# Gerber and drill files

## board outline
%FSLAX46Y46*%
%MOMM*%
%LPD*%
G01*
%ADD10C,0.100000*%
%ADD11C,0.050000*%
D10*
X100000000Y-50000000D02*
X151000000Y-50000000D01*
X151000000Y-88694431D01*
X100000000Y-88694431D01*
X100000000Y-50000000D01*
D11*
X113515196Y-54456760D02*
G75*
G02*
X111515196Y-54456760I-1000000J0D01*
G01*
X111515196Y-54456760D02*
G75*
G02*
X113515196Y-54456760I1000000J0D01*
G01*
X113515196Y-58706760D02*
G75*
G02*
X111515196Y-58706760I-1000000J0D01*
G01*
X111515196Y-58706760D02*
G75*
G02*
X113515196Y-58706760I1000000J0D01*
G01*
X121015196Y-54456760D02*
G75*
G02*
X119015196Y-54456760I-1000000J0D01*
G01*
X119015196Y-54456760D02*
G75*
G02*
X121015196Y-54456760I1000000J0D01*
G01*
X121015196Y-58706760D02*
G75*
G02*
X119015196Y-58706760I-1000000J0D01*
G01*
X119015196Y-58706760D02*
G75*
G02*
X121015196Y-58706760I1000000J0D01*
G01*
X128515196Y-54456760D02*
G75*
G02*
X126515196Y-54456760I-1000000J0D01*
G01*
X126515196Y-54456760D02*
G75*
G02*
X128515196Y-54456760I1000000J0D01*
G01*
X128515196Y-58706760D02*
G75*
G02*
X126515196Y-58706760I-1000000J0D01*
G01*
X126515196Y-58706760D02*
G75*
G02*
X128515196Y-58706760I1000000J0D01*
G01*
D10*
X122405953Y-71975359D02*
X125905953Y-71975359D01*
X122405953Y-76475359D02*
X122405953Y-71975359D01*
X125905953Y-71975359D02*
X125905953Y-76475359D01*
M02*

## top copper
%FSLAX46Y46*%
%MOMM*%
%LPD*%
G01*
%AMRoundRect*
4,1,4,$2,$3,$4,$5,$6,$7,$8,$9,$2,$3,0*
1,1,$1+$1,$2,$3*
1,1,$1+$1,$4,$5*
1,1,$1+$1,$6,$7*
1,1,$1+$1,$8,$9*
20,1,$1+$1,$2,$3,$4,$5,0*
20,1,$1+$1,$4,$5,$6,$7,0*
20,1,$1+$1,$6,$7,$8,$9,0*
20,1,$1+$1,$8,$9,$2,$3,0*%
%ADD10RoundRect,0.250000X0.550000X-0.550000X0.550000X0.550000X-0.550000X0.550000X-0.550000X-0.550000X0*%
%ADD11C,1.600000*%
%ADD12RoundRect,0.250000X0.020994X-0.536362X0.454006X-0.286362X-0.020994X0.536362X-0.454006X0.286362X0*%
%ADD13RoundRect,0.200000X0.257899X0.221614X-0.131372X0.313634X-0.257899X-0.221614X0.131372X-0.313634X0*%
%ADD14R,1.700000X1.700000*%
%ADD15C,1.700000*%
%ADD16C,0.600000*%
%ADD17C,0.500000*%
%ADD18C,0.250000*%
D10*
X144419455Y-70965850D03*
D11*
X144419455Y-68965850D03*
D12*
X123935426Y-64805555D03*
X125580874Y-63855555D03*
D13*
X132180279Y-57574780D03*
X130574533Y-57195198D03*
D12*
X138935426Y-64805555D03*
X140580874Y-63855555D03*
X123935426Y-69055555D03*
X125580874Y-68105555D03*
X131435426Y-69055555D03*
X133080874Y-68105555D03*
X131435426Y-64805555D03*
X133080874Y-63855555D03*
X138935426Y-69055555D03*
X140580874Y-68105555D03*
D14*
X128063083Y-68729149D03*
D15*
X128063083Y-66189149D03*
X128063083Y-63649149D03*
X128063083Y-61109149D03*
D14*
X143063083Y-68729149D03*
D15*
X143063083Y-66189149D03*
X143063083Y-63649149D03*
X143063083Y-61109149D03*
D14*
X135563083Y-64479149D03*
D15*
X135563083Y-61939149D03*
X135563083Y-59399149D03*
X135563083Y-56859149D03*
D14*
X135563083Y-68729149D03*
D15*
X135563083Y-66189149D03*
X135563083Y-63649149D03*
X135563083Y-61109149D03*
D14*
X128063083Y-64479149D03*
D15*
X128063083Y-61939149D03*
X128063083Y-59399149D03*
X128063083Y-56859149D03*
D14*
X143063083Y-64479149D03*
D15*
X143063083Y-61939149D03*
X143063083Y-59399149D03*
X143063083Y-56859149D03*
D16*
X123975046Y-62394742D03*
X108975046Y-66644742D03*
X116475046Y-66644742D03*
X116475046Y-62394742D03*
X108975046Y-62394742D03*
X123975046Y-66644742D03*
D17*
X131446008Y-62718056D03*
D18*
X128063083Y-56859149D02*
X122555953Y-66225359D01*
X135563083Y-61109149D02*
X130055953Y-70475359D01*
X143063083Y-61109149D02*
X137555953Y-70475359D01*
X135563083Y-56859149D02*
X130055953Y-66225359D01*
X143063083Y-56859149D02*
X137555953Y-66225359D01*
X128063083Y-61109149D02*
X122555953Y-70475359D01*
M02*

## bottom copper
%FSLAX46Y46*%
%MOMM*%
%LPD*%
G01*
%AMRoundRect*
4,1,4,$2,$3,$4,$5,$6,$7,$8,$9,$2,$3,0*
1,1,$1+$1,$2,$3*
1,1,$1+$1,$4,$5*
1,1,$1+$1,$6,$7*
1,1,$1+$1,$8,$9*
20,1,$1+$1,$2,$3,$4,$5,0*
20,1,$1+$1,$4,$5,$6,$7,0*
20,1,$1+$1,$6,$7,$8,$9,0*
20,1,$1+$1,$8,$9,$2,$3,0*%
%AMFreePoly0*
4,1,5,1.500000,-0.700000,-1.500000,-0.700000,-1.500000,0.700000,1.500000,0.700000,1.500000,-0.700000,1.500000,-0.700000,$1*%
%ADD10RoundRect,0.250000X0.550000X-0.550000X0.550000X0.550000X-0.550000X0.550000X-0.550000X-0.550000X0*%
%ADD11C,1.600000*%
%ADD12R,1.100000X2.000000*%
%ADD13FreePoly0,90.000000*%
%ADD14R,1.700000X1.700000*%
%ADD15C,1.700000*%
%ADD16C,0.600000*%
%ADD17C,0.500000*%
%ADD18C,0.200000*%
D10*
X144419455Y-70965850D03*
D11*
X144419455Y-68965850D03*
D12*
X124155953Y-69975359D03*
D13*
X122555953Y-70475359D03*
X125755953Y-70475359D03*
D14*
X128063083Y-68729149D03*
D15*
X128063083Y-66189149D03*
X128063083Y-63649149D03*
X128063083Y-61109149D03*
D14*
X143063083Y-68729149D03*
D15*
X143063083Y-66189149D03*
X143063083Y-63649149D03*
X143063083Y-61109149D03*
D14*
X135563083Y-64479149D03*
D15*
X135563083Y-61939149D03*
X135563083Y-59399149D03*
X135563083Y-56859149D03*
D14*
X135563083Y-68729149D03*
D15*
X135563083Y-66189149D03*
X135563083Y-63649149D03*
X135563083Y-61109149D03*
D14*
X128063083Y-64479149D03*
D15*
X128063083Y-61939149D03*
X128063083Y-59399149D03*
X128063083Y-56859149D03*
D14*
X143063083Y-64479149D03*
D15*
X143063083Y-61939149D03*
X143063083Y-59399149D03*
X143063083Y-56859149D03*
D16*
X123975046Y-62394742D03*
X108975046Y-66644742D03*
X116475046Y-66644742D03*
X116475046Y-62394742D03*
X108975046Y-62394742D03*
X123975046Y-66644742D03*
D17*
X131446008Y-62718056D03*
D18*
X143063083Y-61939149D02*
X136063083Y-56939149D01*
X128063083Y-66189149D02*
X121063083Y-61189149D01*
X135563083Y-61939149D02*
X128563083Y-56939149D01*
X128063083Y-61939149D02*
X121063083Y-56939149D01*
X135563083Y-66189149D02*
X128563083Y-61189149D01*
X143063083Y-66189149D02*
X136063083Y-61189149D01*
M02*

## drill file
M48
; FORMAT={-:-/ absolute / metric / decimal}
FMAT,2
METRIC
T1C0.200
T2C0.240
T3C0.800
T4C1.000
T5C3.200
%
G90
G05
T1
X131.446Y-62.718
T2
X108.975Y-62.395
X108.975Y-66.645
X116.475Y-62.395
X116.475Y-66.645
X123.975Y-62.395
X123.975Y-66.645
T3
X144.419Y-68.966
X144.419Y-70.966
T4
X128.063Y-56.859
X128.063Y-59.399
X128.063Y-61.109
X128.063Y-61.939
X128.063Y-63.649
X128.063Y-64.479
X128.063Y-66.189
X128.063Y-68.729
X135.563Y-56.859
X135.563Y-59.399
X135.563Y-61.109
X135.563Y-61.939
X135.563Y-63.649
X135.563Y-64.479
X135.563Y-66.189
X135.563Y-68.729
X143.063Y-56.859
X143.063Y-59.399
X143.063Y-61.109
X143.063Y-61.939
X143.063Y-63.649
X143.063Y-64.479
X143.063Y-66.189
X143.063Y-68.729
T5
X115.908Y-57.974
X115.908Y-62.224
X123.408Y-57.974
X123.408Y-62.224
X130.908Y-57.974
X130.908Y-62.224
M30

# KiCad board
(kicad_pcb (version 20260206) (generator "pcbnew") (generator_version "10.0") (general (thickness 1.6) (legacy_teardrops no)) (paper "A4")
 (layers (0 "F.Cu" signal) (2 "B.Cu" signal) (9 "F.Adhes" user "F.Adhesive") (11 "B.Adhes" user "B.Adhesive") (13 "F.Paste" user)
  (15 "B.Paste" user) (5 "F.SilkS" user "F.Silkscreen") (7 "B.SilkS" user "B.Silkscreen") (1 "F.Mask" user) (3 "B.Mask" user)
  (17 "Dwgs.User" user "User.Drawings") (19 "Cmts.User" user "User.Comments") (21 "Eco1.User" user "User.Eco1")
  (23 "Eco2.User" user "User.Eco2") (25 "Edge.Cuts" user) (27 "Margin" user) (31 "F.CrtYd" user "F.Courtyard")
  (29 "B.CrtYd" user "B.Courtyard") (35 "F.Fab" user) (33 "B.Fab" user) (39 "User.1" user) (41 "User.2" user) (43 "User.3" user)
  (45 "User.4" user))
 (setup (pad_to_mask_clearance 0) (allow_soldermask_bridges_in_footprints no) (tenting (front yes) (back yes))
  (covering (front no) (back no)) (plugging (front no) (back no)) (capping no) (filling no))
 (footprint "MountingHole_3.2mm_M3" (layer "F.Cu") (at 130.908484 62.224067 45)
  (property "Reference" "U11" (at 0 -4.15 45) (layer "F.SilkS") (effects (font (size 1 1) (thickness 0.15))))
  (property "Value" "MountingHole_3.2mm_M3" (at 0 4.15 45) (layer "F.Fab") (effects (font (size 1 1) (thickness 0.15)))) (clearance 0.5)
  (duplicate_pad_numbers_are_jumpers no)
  (pad "" np_thru_hole circle (at 0 0 45) (size 3.2 3.2) (drill 3.2) (layers "*.Cu" "*.Mask")))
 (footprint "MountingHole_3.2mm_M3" (layer "F.Cu") (at 123.408484 62.224067 45)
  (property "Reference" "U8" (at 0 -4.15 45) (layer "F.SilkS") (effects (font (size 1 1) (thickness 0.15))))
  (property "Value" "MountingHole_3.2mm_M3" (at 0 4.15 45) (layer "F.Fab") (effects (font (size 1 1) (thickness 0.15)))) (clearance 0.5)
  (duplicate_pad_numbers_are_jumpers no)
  (pad "" np_thru_hole circle (at 0 0 45) (size 3.2 3.2) (drill 3.2) (layers "*.Cu" "*.Mask")))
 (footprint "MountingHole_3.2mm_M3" (layer "F.Cu") (at 115.908484 62.224067 45)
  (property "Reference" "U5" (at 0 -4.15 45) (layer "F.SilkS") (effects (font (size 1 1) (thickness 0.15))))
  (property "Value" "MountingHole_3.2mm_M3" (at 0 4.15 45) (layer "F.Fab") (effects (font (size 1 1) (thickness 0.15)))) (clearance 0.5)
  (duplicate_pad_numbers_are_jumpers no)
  (pad "" np_thru_hole circle (at 0 0 45) (size 3.2 3.2) (drill 3.2) (layers "*.Cu" "*.Mask")))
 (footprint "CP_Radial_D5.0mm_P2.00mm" (layer "F.Cu") (at 144.419455 70.96585 90)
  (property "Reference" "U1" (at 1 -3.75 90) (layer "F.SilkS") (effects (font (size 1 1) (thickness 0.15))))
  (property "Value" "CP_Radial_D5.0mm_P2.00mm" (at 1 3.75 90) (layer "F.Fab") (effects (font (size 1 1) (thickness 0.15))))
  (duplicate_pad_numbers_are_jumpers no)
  (pad "1" thru_hole roundrect (at 0 0 90) (size 1.6 1.6) (drill 0.8) (layers "*.Cu" "*.Mask") (remove_unused_layers no)
   (roundrect_rratio 0.15625) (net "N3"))
  (pad "2" thru_hole circle (at 2 0 90) (size 1.6 1.6) (drill 0.8) (layers "*.Cu" "*.Mask") (remove_unused_layers no) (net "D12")))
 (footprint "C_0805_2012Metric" (layer "F.Cu") (at 124.75815 64.330555 30)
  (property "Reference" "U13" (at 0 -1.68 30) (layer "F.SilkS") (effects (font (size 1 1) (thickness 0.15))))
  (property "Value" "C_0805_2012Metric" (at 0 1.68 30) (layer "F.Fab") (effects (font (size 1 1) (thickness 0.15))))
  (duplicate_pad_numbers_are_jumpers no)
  (pad "1" smd roundrect (at -0.95 0 30) (size 1 1.45) (layers "F.Cu" "F.Mask" "F.Paste") (roundrect_rratio 0.25) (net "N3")
   (clearance 0.35))
  (pad "2" smd roundrect (at 0.95 0 30) (size 1 1.45) (layers "F.Cu" "F.Mask" "F.Paste") (roundrect_rratio 0.25)))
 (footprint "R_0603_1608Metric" (layer "F.Cu") (at 131.377406 57.384989 166.7)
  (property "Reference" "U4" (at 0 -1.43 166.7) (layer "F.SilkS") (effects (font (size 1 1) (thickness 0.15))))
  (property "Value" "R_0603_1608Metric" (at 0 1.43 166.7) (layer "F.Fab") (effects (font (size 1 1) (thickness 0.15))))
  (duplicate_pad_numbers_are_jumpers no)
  (pad "1" smd roundrect (at -0.825 0 166.7) (size 0.8 0.95) (layers "F.Cu" "F.Mask" "F.Paste") (roundrect_rratio 0.25) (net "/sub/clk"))
  (pad "2" smd roundrect (at 0.825 0 166.7) (size 0.8 0.95) (layers "F.Cu" "F.Mask" "F.Paste") (roundrect_rratio 0.25) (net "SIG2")))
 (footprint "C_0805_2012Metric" (layer "F.Cu") (at 139.75815 64.330555 30)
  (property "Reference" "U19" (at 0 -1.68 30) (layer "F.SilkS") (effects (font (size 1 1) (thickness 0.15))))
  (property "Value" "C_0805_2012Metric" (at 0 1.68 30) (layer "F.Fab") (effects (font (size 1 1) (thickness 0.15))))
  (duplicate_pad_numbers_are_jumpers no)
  (pad "1" smd roundrect (at -0.95 0 30) (size 1 1.45) (layers "F.Cu" "F.Mask" "F.Paste") (roundrect_rratio 0.25) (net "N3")
   (clearance 0.35))
  (pad "2" smd roundrect (at 0.95 0 30) (size 1 1.45) (layers "F.Cu" "F.Mask" "F.Paste") (roundrect_rratio 0.25)))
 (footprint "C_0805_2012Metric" (layer "F.Cu") (at 124.75815 68.580555 30)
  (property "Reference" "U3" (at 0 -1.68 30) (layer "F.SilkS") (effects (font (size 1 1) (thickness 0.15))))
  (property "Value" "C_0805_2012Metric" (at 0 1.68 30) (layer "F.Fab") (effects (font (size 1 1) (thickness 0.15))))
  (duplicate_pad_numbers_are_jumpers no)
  (pad "1" smd roundrect (at -0.95 0 30) (size 1 1.45) (layers "F.Cu" "F.Mask" "F.Paste") (roundrect_rratio 0.25) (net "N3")
   (clearance 0.35))
  (pad "2" smd roundrect (at 0.95 0 30) (size 1 1.45) (layers "F.Cu" "F.Mask" "F.Paste") (roundrect_rratio 0.25)))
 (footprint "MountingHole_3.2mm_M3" (layer "F.Cu") (at 123.408484 57.974067 45)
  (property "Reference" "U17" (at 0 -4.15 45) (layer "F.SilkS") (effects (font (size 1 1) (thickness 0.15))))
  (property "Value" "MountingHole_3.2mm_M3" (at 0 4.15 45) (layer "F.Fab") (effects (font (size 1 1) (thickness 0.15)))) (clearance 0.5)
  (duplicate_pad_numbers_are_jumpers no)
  (pad "" np_thru_hole circle (at 0 0 45) (size 3.2 3.2) (drill 3.2) (layers "*.Cu" "*.Mask")))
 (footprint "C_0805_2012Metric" (layer "F.Cu") (at 132.25815 68.580555 30)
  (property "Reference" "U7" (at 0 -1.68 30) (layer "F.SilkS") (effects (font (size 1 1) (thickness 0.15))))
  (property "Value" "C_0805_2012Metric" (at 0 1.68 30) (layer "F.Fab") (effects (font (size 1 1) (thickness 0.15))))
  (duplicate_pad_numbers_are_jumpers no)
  (pad "1" smd roundrect (at -0.95 0 30) (size 1 1.45) (layers "F.Cu" "F.Mask" "F.Paste") (roundrect_rratio 0.25) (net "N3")
   (clearance 0.35))
  (pad "2" smd roundrect (at 0.95 0 30) (size 1 1.45) (layers "F.Cu" "F.Mask" "F.Paste") (roundrect_rratio 0.25)))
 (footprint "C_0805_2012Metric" (layer "F.Cu") (at 132.25815 64.330555 30)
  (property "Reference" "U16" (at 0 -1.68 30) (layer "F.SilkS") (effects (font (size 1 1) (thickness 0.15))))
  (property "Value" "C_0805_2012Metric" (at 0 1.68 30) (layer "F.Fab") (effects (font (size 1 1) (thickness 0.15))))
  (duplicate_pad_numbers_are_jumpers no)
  (pad "1" smd roundrect (at -0.95 0 30) (size 1 1.45) (layers "F.Cu" "F.Mask" "F.Paste") (roundrect_rratio 0.25) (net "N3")
   (clearance 0.35))
  (pad "2" smd roundrect (at 0.95 0 30) (size 1 1.45) (layers "F.Cu" "F.Mask" "F.Paste") (roundrect_rratio 0.25)))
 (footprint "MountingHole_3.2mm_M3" (layer "F.Cu") (at 115.908484 57.974067 45)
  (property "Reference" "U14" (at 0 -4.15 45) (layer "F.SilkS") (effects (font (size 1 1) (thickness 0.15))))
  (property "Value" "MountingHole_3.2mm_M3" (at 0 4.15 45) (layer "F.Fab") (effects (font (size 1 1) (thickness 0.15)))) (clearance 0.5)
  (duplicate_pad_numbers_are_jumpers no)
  (pad "" np_thru_hole circle (at 0 0 45) (size 3.2 3.2) (drill 3.2) (layers "*.Cu" "*.Mask")))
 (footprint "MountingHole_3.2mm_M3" (layer "F.Cu") (at 130.908484 57.974067 45)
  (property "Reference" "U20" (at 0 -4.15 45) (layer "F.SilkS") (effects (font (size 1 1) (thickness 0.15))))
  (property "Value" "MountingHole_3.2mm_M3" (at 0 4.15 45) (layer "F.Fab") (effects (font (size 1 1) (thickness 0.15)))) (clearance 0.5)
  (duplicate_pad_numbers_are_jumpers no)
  (pad "" np_thru_hole circle (at 0 0 45) (size 3.2 3.2) (drill 3.2) (layers "*.Cu" "*.Mask")))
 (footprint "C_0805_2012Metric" (layer "F.Cu") (at 139.75815 68.580555 30)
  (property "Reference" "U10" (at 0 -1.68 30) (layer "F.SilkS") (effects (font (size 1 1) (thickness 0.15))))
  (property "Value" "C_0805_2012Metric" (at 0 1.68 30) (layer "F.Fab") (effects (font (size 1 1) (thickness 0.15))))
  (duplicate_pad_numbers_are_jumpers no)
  (pad "1" smd roundrect (at -0.95 0 30) (size 1 1.45) (layers "F.Cu" "F.Mask" "F.Paste") (roundrect_rratio 0.25) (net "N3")
   (clearance 0.35))
  (pad "2" smd roundrect (at 0.95 0 30) (size 1 1.45) (layers "F.Cu" "F.Mask" "F.Paste") (roundrect_rratio 0.25)))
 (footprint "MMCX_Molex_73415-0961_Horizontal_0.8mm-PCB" (layer "B.Cu") (at 124.155953 72.725359 90)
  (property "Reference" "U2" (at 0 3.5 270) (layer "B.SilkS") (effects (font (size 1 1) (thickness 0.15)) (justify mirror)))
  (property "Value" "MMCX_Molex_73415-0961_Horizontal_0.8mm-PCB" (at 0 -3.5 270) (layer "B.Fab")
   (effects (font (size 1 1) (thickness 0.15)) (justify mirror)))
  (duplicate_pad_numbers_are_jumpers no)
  (fp_line (start 0.75 -1.75) (end 0.75 1.75) (stroke (width 0.1) (type solid)) (layer "Edge.Cuts"))
  (fp_line (start -3.75 -1.75) (end 0.75 -1.75) (stroke (width 0.1) (type solid)) (layer "Edge.Cuts"))
  (fp_line (start 0.75 1.75) (end -3.75 1.75) (stroke (width 0.1) (type solid)) (layer "Edge.Cuts"))
  (pad "1" smd rect (at 2.75 0 90) (size 2 1.1) (layers "B.Cu" "B.Mask" "B.Paste") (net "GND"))
  (pad "2" smd custom (at 2.25 -1.6 90) (size 3 1.4) (layers "B.Cu" "B.Mask" "B.Paste") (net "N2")
   (options (clearance outline) (anchor rect)) (primitives))
  (pad "2" smd custom (at 2.25 1.6 90) (size 3 1.4) (layers "B.Cu" "B.Mask" "B.Paste") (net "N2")
   (options (clearance outline) (anchor rect)) (primitives)))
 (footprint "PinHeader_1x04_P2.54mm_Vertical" (layer "B.Cu") (at 128.063083 68.729149)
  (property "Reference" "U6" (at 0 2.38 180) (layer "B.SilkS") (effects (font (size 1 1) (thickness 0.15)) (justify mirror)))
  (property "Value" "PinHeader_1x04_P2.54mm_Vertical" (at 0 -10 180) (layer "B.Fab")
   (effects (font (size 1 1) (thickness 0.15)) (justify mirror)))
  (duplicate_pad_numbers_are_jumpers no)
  (pad "1" thru_hole rect (at 0 0) (size 1.7 1.7) (drill 1) (layers "*.Cu" "*.Mask") (remove_unused_layers no) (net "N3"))
  (pad "2" thru_hole circle (at 0 -2.54) (size 1.7 1.7) (drill 1) (layers "*.Cu" "*.Mask") (remove_unused_layers no) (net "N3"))
  (pad "3" thru_hole circle (at 0 -5.08) (size 1.7 1.7) (drill 1) (layers "*.Cu" "*.Mask") (remove_unused_layers no) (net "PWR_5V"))
  (pad "4" thru_hole circle (at 0 -7.62) (size 1.7 1.7) (drill 1) (layers "*.Cu" "*.Mask") (remove_unused_layers no)))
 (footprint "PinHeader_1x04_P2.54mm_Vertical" (layer "B.Cu") (at 143.063083 68.729149)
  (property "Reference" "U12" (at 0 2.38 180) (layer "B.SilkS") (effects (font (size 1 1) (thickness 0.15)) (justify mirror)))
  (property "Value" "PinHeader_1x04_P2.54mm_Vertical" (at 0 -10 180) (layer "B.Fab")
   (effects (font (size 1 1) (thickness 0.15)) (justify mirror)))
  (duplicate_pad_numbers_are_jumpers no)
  (pad "1" thru_hole rect (at 0 0) (size 1.7 1.7) (drill 1) (layers "*.Cu" "*.Mask") (remove_unused_layers no) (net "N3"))
  (pad "2" thru_hole circle (at 0 -2.54) (size 1.7 1.7) (drill 1) (layers "*.Cu" "*.Mask") (remove_unused_layers no) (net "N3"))
  (pad "3" thru_hole circle (at 0 -5.08) (size 1.7 1.7) (drill 1) (layers "*.Cu" "*.Mask") (remove_unused_layers no) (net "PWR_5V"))
  (pad "4" thru_hole circle (at 0 -7.62) (size 1.7 1.7) (drill 1) (layers "*.Cu" "*.Mask") (remove_unused_layers no)))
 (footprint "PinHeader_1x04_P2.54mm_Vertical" (layer "B.Cu") (at 135.563083 64.479149)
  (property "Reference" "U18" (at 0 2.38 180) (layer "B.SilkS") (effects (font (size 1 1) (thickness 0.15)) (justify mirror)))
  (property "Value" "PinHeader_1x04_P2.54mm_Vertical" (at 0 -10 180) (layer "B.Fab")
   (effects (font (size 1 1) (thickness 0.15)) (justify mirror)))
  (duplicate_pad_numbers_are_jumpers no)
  (pad "1" thru_hole rect (at 0 0) (size 1.7 1.7) (drill 1) (layers "*.Cu" "*.Mask") (remove_unused_layers no) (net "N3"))
  (pad "2" thru_hole circle (at 0 -2.54) (size 1.7 1.7) (drill 1) (layers "*.Cu" "*.Mask") (remove_unused_layers no) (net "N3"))
  (pad "3" thru_hole circle (at 0 -5.08) (size 1.7 1.7) (drill 1) (layers "*.Cu" "*.Mask") (remove_unused_layers no) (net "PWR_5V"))
  (pad "4" thru_hole circle (at 0 -7.62) (size 1.7 1.7) (drill 1) (layers "*.Cu" "*.Mask") (remove_unused_layers no)))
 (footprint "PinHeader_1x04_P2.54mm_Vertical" (layer "B.Cu") (at 135.563083 68.729149)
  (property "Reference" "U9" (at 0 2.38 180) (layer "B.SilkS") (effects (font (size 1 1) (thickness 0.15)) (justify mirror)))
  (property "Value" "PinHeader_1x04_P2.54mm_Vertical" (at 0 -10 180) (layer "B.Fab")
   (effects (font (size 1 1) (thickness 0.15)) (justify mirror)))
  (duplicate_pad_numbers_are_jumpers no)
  (pad "1" thru_hole rect (at 0 0) (size 1.7 1.7) (drill 1) (layers "*.Cu" "*.Mask") (remove_unused_layers no) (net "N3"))
  (pad "2" thru_hole circle (at 0 -2.54) (size 1.7 1.7) (drill 1) (layers "*.Cu" "*.Mask") (remove_unused_layers no) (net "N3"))
  (pad "3" thru_hole circle (at 0 -5.08) (size 1.7 1.7) (drill 1) (layers "*.Cu" "*.Mask") (remove_unused_layers no) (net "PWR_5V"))
  (pad "4" thru_hole circle (at 0 -7.62) (size 1.7 1.7) (drill 1) (layers "*.Cu" "*.Mask") (remove_unused_layers no)))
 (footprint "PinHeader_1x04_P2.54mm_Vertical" (layer "B.Cu") (at 128.063083 64.479149)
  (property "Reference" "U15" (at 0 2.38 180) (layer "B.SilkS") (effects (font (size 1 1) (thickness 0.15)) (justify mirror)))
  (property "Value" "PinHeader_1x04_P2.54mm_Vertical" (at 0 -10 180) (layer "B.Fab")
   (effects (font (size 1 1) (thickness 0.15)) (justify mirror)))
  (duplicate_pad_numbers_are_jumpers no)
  (pad "1" thru_hole rect (at 0 0) (size 1.7 1.7) (drill 1) (layers "*.Cu" "*.Mask") (remove_unused_layers no) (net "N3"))
  (pad "2" thru_hole circle (at 0 -2.54) (size 1.7 1.7) (drill 1) (layers "*.Cu" "*.Mask") (remove_unused_layers no) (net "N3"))
  (pad "3" thru_hole circle (at 0 -5.08) (size 1.7 1.7) (drill 1) (layers "*.Cu" "*.Mask") (remove_unused_layers no) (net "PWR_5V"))
  (pad "4" thru_hole circle (at 0 -7.62) (size 1.7 1.7) (drill 1) (layers "*.Cu" "*.Mask") (remove_unused_layers no)))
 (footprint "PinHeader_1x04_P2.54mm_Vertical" (layer "B.Cu") (at 143.063083 64.479149)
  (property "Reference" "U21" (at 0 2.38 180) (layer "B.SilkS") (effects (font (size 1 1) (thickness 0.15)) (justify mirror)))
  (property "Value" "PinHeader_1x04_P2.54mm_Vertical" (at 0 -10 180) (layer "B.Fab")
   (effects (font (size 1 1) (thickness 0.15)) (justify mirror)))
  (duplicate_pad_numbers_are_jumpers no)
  (pad "1" thru_hole rect (at 0 0) (size 1.7 1.7) (drill 1) (layers "*.Cu" "*.Mask") (remove_unused_layers no) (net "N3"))
  (pad "2" thru_hole circle (at 0 -2.54) (size 1.7 1.7) (drill 1) (layers "*.Cu" "*.Mask") (remove_unused_layers no) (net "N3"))
  (pad "3" thru_hole circle (at 0 -5.08) (size 1.7 1.7) (drill 1) (layers "*.Cu" "*.Mask") (remove_unused_layers no) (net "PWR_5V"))
  (pad "4" thru_hole circle (at 0 -7.62) (size 1.7 1.7) (drill 1) (layers "*.Cu" "*.Mask") (remove_unused_layers no)))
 (gr_rect (start 100 50) (end 151 88.694431) (stroke (width 0.1) (type default)) (fill no) (layer "Edge.Cuts"))
 (gr_circle (center 112.515196 54.45676) (end 113.515196 54.45676) (stroke (width 0.05) (type default)) (fill no) (layer "Edge.Cuts"))
 (gr_circle (center 112.515196 58.70676) (end 113.515196 58.70676) (stroke (width 0.05) (type default)) (fill no) (layer "Edge.Cuts"))
 (gr_circle (center 120.015196 54.45676) (end 121.015196 54.45676) (stroke (width 0.05) (type default)) (fill no) (layer "Edge.Cuts"))
 (gr_circle (center 120.015196 58.70676) (end 121.015196 58.70676) (stroke (width 0.05) (type default)) (fill no) (layer "Edge.Cuts"))
 (gr_circle (center 127.515196 54.45676) (end 128.515196 54.45676) (stroke (width 0.05) (type default)) (fill no) (layer "Edge.Cuts"))
 (gr_circle (center 127.515196 58.70676) (end 128.515196 58.70676) (stroke (width 0.05) (type default)) (fill no) (layer "Edge.Cuts"))
 (segment (start 128.063083 56.859149) (end 122.555953 66.225359) (width 0.25) (layer "F.Cu") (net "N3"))
 (segment (start 135.563083 61.109149) (end 130.055953 70.475359) (width 0.25) (layer "F.Cu") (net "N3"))
 (segment (start 143.063083 61.109149) (end 137.555953 70.475359) (width 0.25) (layer "F.Cu") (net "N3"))
 (segment (start 135.563083 56.859149) (end 130.055953 66.225359) (width 0.25) (layer "F.Cu") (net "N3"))
 (segment (start 143.063083 56.859149) (end 137.555953 66.225359) (width 0.25) (layer "F.Cu") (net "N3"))
 (segment (start 128.063083 61.109149) (end 122.555953 70.475359) (width 0.25) (layer "F.Cu") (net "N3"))
 (segment (start 143.063083 61.939149) (end 136.063083 56.939149) (width 0.2) (layer "B.Cu") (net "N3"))
 (segment (start 128.063083 66.189149) (end 121.063083 61.189149) (width 0.2) (layer "B.Cu") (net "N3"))
 (segment (start 135.563083 61.939149) (end 128.563083 56.939149) (width 0.2) (layer "B.Cu") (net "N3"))
 (segment (start 128.063083 61.939149) (end 121.063083 56.939149) (width 0.2) (layer "B.Cu") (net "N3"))
 (segment (start 135.563083 66.189149) (end 128.563083 61.189149) (width 0.2) (layer "B.Cu") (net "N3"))
 (segment (start 143.063083 66.189149) (end 136.063083 61.189149) (width 0.2) (layer "B.Cu") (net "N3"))
 (via (at 123.975046 62.394742) (size 0.6) (drill 0.24) (layers "F.Cu" "B.Cu") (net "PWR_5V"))
 (via (at 108.975046 66.644742) (size 0.6) (drill 0.24) (layers "F.Cu" "B.Cu") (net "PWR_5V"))
 (via (at 116.475046 66.644742) (size 0.6) (drill 0.24) (layers "F.Cu" "B.Cu") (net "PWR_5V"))
 (via (at 116.475046 62.394742) (size 0.6) (drill 0.24) (layers "F.Cu" "B.Cu") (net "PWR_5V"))
 (via (at 108.975046 62.394742) (size 0.6) (drill 0.24) (layers "F.Cu" "B.Cu") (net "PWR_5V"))
 (via (at 123.975046 66.644742) (size 0.6) (drill 0.24) (layers "F.Cu" "B.Cu") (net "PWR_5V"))
 (via (at 131.446008 62.718056) (size 0.5) (drill 0.2) (layers "F.Cu" "B.Cu") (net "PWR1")))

